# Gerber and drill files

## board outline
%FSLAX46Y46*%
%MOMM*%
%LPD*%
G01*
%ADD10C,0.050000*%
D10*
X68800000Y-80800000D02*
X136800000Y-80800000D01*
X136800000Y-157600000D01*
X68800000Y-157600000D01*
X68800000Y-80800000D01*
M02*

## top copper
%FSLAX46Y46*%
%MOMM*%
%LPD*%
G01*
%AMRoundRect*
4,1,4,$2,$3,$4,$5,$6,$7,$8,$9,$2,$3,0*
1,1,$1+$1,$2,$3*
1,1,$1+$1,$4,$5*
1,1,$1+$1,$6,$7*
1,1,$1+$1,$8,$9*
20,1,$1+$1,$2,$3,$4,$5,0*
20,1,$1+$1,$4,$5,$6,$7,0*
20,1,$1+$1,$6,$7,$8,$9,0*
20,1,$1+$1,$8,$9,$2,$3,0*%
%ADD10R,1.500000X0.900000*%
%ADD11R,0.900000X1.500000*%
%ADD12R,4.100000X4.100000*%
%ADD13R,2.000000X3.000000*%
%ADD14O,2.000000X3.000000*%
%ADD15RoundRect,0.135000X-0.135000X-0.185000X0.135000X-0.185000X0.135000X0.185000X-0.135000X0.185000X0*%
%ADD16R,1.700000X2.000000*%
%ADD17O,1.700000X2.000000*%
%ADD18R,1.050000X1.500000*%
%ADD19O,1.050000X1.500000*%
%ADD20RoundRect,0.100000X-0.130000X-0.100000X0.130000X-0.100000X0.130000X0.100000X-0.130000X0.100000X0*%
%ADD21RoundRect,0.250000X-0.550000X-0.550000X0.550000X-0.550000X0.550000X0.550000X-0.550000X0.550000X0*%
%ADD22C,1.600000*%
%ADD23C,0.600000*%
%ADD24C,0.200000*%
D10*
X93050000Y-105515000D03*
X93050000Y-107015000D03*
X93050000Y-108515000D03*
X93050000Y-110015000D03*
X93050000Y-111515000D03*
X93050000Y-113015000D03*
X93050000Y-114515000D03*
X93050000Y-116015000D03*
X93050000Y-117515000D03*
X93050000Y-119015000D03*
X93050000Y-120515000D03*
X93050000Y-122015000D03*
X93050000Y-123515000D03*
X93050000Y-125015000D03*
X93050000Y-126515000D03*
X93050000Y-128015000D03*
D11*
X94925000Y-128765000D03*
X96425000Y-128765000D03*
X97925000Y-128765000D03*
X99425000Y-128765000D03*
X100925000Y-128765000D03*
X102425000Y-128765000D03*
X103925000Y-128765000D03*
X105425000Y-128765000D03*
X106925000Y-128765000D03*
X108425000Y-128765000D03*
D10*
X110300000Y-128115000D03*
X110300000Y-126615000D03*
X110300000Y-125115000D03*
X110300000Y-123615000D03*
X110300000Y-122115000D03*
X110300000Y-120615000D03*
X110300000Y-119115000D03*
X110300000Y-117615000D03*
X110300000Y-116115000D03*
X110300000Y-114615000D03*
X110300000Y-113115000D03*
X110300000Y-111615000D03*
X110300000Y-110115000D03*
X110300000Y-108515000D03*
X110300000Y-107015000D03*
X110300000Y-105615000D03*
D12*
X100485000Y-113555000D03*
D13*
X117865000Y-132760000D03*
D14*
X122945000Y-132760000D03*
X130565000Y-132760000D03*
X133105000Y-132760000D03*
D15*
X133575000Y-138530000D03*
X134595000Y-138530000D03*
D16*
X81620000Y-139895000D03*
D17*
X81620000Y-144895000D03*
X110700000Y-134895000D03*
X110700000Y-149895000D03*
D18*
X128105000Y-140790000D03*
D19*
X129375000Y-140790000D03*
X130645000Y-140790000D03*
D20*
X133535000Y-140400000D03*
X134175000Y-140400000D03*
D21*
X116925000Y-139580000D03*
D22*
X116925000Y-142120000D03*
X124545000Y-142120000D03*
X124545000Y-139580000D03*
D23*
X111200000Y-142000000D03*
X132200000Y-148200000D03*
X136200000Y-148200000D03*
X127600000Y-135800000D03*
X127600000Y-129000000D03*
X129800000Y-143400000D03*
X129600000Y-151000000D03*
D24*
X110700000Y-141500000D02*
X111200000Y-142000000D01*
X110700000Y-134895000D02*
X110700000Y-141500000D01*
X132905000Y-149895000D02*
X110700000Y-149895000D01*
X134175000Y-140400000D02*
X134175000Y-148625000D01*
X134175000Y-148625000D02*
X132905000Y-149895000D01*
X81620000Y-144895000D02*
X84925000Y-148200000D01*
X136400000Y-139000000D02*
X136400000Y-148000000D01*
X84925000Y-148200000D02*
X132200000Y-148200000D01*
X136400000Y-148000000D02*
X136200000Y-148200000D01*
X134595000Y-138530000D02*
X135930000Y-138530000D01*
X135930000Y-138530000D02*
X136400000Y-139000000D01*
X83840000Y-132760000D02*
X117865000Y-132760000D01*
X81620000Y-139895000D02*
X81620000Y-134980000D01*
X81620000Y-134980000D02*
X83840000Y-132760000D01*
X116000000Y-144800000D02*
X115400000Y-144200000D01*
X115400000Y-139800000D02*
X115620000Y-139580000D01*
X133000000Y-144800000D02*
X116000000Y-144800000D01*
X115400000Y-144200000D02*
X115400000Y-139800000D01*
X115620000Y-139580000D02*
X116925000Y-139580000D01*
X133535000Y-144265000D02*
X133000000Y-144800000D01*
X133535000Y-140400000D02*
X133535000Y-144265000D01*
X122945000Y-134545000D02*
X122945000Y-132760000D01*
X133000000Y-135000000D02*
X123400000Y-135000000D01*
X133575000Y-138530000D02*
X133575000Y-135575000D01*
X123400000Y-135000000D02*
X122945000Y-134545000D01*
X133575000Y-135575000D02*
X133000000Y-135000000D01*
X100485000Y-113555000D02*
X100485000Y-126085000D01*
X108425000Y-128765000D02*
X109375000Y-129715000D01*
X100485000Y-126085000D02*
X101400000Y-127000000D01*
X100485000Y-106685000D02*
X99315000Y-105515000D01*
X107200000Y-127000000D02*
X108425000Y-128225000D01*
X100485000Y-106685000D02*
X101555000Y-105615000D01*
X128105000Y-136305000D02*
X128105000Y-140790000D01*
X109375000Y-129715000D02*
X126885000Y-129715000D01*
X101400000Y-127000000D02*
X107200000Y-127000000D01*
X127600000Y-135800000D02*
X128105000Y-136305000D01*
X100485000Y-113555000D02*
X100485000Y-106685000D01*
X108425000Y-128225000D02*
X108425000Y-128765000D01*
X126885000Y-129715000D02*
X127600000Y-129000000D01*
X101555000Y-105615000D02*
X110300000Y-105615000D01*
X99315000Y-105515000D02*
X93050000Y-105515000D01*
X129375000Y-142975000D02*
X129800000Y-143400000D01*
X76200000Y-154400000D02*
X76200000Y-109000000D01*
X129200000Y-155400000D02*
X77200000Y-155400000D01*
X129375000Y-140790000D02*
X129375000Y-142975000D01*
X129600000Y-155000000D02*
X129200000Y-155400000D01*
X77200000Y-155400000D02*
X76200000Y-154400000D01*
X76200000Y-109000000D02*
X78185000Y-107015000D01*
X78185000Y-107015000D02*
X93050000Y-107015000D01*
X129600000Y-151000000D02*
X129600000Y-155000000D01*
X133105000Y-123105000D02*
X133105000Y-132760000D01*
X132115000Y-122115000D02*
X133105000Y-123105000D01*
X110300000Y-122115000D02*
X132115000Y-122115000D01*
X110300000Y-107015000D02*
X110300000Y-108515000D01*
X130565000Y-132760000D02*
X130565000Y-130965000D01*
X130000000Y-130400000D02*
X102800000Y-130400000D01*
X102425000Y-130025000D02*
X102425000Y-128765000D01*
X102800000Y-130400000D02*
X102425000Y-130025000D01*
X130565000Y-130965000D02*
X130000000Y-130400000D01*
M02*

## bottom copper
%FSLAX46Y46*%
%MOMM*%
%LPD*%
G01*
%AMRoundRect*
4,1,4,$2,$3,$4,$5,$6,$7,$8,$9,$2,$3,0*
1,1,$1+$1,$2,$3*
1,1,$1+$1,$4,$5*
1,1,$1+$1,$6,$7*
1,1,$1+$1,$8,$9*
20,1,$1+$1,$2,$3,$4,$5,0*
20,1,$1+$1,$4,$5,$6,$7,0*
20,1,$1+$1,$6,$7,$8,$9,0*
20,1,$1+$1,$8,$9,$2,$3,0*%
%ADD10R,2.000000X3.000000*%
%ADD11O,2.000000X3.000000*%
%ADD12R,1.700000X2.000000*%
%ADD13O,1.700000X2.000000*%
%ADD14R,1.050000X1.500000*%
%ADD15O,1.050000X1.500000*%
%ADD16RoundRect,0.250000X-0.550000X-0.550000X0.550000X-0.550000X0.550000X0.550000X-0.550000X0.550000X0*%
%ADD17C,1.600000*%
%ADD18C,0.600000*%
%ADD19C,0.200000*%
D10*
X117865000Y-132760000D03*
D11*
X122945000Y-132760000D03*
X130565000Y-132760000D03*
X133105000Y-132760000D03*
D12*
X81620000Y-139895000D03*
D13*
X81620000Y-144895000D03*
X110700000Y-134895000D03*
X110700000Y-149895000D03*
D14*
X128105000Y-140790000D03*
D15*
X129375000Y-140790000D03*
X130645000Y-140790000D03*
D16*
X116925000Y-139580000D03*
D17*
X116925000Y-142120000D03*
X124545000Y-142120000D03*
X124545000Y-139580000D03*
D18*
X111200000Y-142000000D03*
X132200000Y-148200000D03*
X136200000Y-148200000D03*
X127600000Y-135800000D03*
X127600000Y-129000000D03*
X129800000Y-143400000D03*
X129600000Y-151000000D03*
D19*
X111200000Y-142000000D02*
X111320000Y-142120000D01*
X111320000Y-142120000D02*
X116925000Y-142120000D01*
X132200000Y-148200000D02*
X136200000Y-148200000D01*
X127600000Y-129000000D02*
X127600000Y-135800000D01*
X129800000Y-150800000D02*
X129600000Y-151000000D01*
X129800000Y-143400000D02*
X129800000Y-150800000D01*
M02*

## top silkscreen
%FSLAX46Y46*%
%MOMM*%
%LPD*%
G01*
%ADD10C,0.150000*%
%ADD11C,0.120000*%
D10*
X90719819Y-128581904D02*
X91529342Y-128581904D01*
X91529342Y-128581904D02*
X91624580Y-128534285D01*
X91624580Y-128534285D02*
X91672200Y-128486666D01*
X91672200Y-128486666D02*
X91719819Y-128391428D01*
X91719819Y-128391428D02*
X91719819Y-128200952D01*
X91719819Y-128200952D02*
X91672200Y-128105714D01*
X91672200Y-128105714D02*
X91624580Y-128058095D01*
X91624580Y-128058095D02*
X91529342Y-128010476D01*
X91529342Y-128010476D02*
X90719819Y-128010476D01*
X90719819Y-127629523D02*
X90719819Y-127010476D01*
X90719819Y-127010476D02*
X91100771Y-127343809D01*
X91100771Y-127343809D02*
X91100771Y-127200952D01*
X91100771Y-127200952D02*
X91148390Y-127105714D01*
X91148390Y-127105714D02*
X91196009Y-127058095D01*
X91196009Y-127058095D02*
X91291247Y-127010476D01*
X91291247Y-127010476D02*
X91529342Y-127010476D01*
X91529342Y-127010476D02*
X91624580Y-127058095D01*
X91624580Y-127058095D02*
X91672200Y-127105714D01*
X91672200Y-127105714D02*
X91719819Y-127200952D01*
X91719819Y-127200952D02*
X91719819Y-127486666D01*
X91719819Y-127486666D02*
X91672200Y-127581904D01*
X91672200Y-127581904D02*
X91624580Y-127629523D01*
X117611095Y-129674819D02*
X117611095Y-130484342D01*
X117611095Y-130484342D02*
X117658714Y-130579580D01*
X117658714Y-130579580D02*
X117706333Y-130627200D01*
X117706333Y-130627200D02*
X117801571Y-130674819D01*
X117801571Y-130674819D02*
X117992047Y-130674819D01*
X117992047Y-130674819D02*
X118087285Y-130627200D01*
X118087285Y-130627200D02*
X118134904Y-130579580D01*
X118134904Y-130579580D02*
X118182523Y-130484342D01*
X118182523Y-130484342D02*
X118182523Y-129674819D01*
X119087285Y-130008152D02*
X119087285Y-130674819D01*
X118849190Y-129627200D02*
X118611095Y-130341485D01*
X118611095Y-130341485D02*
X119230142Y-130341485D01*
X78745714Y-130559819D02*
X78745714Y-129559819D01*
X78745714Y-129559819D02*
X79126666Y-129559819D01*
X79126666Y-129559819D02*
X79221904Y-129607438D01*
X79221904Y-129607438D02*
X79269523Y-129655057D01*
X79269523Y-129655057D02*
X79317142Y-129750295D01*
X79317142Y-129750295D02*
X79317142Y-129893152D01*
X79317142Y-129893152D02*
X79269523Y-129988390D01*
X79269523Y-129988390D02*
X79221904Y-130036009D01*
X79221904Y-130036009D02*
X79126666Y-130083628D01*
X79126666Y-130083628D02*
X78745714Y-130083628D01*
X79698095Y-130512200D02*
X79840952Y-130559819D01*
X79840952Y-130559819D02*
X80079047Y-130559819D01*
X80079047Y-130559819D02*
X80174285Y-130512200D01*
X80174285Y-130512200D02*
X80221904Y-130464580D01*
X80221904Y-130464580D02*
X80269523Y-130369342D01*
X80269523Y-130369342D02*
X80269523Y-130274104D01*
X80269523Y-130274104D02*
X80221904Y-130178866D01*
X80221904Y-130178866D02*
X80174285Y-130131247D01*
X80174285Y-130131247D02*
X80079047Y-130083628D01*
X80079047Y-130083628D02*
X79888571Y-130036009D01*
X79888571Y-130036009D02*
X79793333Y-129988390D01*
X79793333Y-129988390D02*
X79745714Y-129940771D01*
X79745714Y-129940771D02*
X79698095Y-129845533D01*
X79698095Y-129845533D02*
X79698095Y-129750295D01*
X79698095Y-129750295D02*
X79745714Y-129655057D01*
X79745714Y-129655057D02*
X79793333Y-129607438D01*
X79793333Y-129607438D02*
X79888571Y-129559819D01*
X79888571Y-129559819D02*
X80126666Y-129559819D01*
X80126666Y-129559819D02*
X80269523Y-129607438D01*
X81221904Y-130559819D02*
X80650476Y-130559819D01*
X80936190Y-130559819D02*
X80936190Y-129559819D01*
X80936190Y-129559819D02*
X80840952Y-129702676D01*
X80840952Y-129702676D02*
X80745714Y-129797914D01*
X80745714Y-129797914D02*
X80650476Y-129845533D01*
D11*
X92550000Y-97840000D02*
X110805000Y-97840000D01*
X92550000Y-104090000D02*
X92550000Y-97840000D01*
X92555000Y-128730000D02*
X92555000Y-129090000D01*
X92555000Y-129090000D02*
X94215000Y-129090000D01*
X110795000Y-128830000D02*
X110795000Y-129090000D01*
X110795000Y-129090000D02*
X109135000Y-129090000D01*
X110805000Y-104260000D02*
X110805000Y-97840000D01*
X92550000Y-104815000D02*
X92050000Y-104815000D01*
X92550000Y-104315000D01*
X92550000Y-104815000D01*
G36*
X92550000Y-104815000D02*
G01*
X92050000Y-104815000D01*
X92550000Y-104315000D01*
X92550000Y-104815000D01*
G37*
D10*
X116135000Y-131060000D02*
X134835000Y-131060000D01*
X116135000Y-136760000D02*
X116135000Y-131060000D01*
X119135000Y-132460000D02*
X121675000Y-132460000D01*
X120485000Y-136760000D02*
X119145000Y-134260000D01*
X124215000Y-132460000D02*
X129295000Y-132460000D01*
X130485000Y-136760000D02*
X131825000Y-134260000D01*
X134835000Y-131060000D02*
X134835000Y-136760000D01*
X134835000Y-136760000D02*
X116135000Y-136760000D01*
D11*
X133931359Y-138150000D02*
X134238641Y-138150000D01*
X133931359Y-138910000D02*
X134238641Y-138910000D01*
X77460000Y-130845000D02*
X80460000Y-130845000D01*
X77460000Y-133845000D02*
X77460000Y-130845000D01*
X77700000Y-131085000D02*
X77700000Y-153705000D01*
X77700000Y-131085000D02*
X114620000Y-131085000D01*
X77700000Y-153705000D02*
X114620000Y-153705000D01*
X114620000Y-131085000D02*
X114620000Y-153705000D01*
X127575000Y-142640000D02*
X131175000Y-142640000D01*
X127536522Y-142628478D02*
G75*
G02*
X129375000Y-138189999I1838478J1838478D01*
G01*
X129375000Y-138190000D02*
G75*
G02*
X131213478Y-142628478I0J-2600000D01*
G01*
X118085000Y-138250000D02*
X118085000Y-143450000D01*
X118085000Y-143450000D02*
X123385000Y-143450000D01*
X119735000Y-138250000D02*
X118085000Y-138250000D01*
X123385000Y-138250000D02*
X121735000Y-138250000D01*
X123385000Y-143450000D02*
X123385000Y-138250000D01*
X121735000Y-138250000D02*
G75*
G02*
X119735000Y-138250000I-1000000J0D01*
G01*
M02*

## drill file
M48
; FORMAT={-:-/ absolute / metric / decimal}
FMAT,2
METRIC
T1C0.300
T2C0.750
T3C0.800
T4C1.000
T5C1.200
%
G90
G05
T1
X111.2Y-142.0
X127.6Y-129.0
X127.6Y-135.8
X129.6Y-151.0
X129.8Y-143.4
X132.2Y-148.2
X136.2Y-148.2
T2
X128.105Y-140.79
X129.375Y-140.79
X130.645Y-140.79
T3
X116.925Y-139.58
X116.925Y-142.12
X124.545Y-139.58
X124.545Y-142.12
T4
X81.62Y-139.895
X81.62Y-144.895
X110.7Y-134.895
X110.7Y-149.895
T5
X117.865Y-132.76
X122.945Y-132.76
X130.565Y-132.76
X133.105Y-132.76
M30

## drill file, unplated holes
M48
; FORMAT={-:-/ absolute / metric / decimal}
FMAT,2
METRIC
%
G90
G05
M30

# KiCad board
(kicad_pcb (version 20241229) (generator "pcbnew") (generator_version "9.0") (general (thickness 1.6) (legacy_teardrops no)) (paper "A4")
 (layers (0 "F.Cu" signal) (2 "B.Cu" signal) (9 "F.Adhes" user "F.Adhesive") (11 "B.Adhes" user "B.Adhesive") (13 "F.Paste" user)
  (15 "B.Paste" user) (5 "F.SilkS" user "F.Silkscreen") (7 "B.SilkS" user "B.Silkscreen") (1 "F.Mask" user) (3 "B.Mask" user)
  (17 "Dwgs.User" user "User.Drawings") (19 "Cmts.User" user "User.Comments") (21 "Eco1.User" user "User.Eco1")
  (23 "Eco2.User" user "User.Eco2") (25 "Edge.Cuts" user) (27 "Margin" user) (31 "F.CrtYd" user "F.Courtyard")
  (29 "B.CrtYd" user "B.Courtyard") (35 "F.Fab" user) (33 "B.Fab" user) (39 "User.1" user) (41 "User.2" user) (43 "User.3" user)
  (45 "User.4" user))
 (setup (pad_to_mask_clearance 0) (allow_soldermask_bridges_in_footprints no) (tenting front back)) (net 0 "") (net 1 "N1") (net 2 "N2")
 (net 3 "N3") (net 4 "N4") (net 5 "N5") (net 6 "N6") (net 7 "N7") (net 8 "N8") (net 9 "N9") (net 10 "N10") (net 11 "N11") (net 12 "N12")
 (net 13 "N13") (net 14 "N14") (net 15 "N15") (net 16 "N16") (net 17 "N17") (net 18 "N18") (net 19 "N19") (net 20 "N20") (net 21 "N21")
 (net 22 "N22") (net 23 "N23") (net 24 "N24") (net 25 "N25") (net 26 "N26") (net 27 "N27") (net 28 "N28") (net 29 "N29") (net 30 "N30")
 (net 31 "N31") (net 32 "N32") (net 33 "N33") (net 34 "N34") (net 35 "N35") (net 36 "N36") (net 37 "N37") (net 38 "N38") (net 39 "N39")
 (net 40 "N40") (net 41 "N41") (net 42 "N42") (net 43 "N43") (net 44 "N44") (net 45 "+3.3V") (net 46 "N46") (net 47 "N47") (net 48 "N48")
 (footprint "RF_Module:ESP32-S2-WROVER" (layer "F.Cu") (at 101.675 117.29)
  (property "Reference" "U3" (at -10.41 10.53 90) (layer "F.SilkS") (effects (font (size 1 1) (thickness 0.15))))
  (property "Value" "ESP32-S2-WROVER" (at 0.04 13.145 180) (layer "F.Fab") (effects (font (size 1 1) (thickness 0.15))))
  (fp_line (start -9.125 -19.45) (end 9.13 -19.45) (stroke (width 0.12) (type solid)) (layer "F.SilkS"))
  (fp_line (start -9.125 -13.2) (end -9.125 -19.45) (stroke (width 0.12) (type solid)) (layer "F.SilkS"))
  (fp_line (start -9.12 11.44) (end -9.12 11.8) (stroke (width 0.12) (type solid)) (layer "F.SilkS"))
  (fp_line (start -9.12 11.8) (end -7.46 11.8) (stroke (width 0.12) (type solid)) (layer "F.SilkS"))
  (fp_line (start 9.12 11.54) (end 9.12 11.8) (stroke (width 0.12) (type solid)) (layer "F.SilkS"))
  (fp_line (start 9.12 11.8) (end 7.46 11.8) (stroke (width 0.12) (type solid)) (layer "F.SilkS"))
  (fp_line (start 9.13 -13.03) (end 9.13 -19.45) (stroke (width 0.12) (type solid)) (layer "F.SilkS"))
  (fp_poly
   (pts (xy -9.125 -12.475) (xy -9.625 -12.475) (xy -9.125 -12.975) (xy -9.125 -12.475)) (stroke (width 0.12) (type solid)) (fill yes)
   (layer "F.SilkS"))
  (pad "" smd roundrect (at -2.52 -5.065) (size 1.07 1.07) (layers "F.Paste") (roundrect_rratio 0.233645))
  (pad "" smd roundrect (at -2.52 -3.735) (size 1.07 1.07) (layers "F.Paste") (roundrect_rratio 0.233645))
  (pad "" smd roundrect (at -2.52 -2.405) (size 1.07 1.07) (layers "F.Paste") (roundrect_rratio 0.233645))
  (pad "" smd roundrect (at -1.19 -5.065) (size 1.07 1.07) (layers "F.Paste") (roundrect_rratio 0.233645))
  (pad "" smd roundrect (at -1.19 -3.735) (size 1.07 1.07) (layers "F.Paste") (roundrect_rratio 0.233645))
  (pad "" smd roundrect (at -1.19 -2.405) (size 1.07 1.07) (layers "F.Paste") (roundrect_rratio 0.233645))
  (pad "" smd roundrect (at 0.14 -5.065) (size 1.07 1.07) (layers "F.Paste") (roundrect_rratio 0.233645))
  (pad "" smd roundrect (at 0.14 -3.735) (size 1.07 1.07) (layers "F.Paste") (roundrect_rratio 0.233645))
  (pad "" smd roundrect (at 0.14 -2.405) (size 1.07 1.07) (layers "F.Paste") (roundrect_rratio 0.233645))
  (pad "1" smd rect (at -8.625 -11.775) (size 1.5 0.9) (layers "F.Cu" "F.Mask" "F.Paste") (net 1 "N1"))
  (pad "2" smd rect (at -8.625 -10.275) (size 1.5 0.9) (layers "F.Cu" "F.Mask" "F.Paste") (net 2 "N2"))
  (pad "3" smd rect (at -8.625 -8.775) (size 1.5 0.9) (layers "F.Cu" "F.Mask" "F.Paste") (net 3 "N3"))
  (pad "4" smd rect (at -8.625 -7.275) (size 1.5 0.9) (layers "F.Cu" "F.Mask" "F.Paste") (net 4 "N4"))
  (pad "5" smd rect (at -8.625 -5.775) (size 1.5 0.9) (layers "F.Cu" "F.Mask" "F.Paste") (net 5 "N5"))
  (pad "6" smd rect (at -8.625 -4.275) (size 1.5 0.9) (layers "F.Cu" "F.Mask" "F.Paste") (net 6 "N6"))
  (pad "7" smd rect (at -8.625 -2.775) (size 1.5 0.9) (layers "F.Cu" "F.Mask" "F.Paste") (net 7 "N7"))
  (pad "8" smd rect (at -8.625 -1.275) (size 1.5 0.9) (layers "F.Cu" "F.Mask" "F.Paste") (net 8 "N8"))
  (pad "9" smd rect (at -8.625 0.225) (size 1.5 0.9) (layers "F.Cu" "F.Mask" "F.Paste") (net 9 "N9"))
  (pad "10" smd rect (at -8.625 1.725) (size 1.5 0.9) (layers "F.Cu" "F.Mask" "F.Paste") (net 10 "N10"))
  (pad "11" smd rect (at -8.625 3.225) (size 1.5 0.9) (layers "F.Cu" "F.Mask" "F.Paste") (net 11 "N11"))
  (pad "12" smd rect (at -8.625 4.725) (size 1.5 0.9) (layers "F.Cu" "F.Mask" "F.Paste") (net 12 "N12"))
  (pad "13" smd rect (at -8.625 6.225) (size 1.5 0.9) (layers "F.Cu" "F.Mask" "F.Paste") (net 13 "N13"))
  (pad "14" smd rect (at -8.625 7.725) (size 1.5 0.9) (layers "F.Cu" "F.Mask" "F.Paste") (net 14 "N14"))
  (pad "15" smd rect (at -8.625 9.225 180) (size 1.5 0.9) (layers "F.Cu" "F.Mask" "F.Paste") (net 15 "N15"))
  (pad "16" smd rect (at -8.625 10.725 180) (size 1.5 0.9) (layers "F.Cu" "F.Mask" "F.Paste") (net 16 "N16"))
  (pad "17" smd rect (at -6.75 11.475) (size 0.9 1.5) (layers "F.Cu" "F.Mask" "F.Paste") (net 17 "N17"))
  (pad "18" smd rect (at -5.25 11.475) (size 0.9 1.5) (layers "F.Cu" "F.Mask" "F.Paste") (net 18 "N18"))
  (pad "19" smd rect (at -3.75 11.475) (size 0.9 1.5) (layers "F.Cu" "F.Mask" "F.Paste") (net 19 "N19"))
  (pad "20" smd rect (at -2.25 11.475) (size 0.9 1.5) (layers "F.Cu" "F.Mask" "F.Paste") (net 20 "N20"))
  (pad "21" smd rect (at -0.75 11.475) (size 0.9 1.5) (layers "F.Cu" "F.Mask" "F.Paste") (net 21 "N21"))
  (pad "22" smd rect (at 0.75 11.475) (size 0.9 1.5) (layers "F.Cu" "F.Mask" "F.Paste") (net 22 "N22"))
  (pad "23" smd rect (at 2.25 11.475) (size 0.9 1.5) (layers "F.Cu" "F.Mask" "F.Paste") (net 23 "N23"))
  (pad "24" smd rect (at 3.75 11.475) (size 0.9 1.5) (layers "F.Cu" "F.Mask" "F.Paste") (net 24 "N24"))
  (pad "25" smd rect (at 5.25 11.475) (size 0.9 1.5) (layers "F.Cu" "F.Mask" "F.Paste") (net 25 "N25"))
  (pad "26" smd rect (at 6.75 11.475) (size 0.9 1.5) (layers "F.Cu" "F.Mask" "F.Paste") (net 1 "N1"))
  (pad "27" smd rect (at 8.625 10.825) (size 1.5 0.9) (layers "F.Cu" "F.Mask" "F.Paste") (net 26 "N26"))
  (pad "28" smd rect (at 8.625 9.325) (size 1.5 0.9) (layers "F.Cu" "F.Mask" "F.Paste") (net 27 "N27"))
  (pad "29" smd rect (at 8.625 7.825) (size 1.5 0.9) (layers "F.Cu" "F.Mask" "F.Paste") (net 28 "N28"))
  (pad "30" smd rect (at 8.625 6.325) (size 1.5 0.9) (layers "F.Cu" "F.Mask" "F.Paste") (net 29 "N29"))
  (pad "31" smd rect (at 8.625 4.825) (size 1.5 0.9) (layers "F.Cu" "F.Mask" "F.Paste") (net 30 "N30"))
  (pad "32" smd rect (at 8.625 3.325) (size 1.5 0.9) (layers "F.Cu" "F.Mask" "F.Paste") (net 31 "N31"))
  (pad "33" smd rect (at 8.625 1.825) (size 1.5 0.9) (layers "F.Cu" "F.Mask" "F.Paste") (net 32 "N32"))
  (pad "34" smd rect (at 8.625 0.325) (size 1.5 0.9) (layers "F.Cu" "F.Mask" "F.Paste") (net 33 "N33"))
  (pad "35" smd rect (at 8.625 -1.175) (size 1.5 0.9) (layers "F.Cu" "F.Mask" "F.Paste") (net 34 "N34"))
  (pad "36" smd rect (at 8.625 -2.675) (size 1.5 0.9) (layers "F.Cu" "F.Mask" "F.Paste") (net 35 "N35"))
  (pad "37" smd rect (at 8.625 -4.175) (size 1.5 0.9) (layers "F.Cu" "F.Mask" "F.Paste") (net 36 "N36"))
  (pad "38" smd rect (at 8.625 -5.675) (size 1.5 0.9) (layers "F.Cu" "F.Mask" "F.Paste") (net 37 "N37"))
  (pad "39" smd rect (at 8.625 -7.175) (size 1.5 0.9) (layers "F.Cu" "F.Mask" "F.Paste") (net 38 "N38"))
  (pad "40" smd rect (at 8.625 -8.775) (size 1.5 0.9) (layers "F.Cu" "F.Mask" "F.Paste") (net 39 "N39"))
  (pad "41" smd rect (at 8.625 -10.275) (size 1.5 0.9) (layers "F.Cu" "F.Mask" "F.Paste") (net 39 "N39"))
  (pad "42" smd rect (at 8.625 -11.675) (size 1.5 0.9) (layers "F.Cu" "F.Mask" "F.Paste") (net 1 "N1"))
  (pad "43" smd rect (at -1.19 -3.735) (size 4.1 4.1) (layers "F.Cu" "F.Mask") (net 1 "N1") (zone_connect 2))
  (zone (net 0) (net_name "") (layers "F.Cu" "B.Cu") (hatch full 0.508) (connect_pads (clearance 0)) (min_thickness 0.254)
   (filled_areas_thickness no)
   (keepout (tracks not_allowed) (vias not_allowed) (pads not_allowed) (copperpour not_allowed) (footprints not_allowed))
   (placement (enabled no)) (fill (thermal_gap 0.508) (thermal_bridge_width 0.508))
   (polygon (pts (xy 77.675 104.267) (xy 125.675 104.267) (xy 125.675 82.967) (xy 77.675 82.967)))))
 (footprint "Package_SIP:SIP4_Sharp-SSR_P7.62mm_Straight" (layer "F.Cu") (at 117.865 132.76)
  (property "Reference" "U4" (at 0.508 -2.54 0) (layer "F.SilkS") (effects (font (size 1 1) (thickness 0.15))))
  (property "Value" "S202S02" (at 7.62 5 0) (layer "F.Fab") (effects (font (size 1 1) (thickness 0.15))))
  (fp_line (start -1.73 -1.7) (end 16.97 -1.7) (stroke (width 0.15) (type solid)) (layer "F.SilkS"))
  (fp_line (start -1.73 4) (end -1.73 -1.7) (stroke (width 0.15) (type solid)) (layer "F.SilkS"))
  (fp_line (start 1.27 -0.3) (end 3.81 -0.3) (stroke (width 0.15) (type solid)) (layer "F.SilkS"))
  (fp_line (start 2.62 4) (end 1.28 1.5) (stroke (width 0.15) (type solid)) (layer "F.SilkS"))
  (fp_line (start 6.35 -0.3) (end 11.43 -0.3) (stroke (width 0.15) (type solid)) (layer "F.SilkS"))
  (fp_line (start 12.62 4) (end 13.96 1.5) (stroke (width 0.15) (type solid)) (layer "F.SilkS"))
  (fp_line (start 16.97 -1.7) (end 16.97 4) (stroke (width 0.15) (type solid)) (layer "F.SilkS"))
  (fp_line (start 16.97 4) (end -1.73 4) (stroke (width 0.15) (type solid)) (layer "F.SilkS"))
  (pad "1" thru_hole rect (at 0 0) (size 2 3) (drill 1.2) (layers "*.Cu" "*.Mask") (remove_unused_layers no) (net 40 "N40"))
  (pad "2" thru_hole oval (at 5.08 0) (size 2 3) (drill 1.2) (layers "*.Cu" "*.Mask") (remove_unused_layers no) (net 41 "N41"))
  (pad "3" thru_hole oval (at 12.7 0) (size 2 3) (drill 1.2) (layers "*.Cu" "*.Mask") (remove_unused_layers no) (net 22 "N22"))
  (pad "4" thru_hole oval (at 15.24 0) (size 2 3) (drill 1.2) (layers "*.Cu" "*.Mask") (remove_unused_layers no) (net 30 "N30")))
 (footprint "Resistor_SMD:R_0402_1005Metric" (layer "F.Cu") (at 134.085 138.53)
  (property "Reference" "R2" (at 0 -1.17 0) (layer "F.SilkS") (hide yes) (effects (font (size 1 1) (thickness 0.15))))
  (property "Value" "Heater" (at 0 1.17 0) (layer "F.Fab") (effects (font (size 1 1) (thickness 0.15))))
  (fp_line (start -0.153641 -0.38) (end 0.153641 -0.38) (stroke (width 0.12) (type solid)) (layer "F.SilkS"))
  (fp_line (start -0.153641 0.38) (end 0.153641 0.38) (stroke (width 0.12) (type solid)) (layer "F.SilkS"))
  (pad "1" smd roundrect (at -0.51 0) (size 0.54 0.64) (layers "F.Cu" "F.Mask" "F.Paste") (roundrect_rratio 0.25) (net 41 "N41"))
  (pad "2" smd roundrect (at 0.51 0) (size 0.54 0.64) (layers "F.Cu" "F.Mask" "F.Paste") (roundrect_rratio 0.25) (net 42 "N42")))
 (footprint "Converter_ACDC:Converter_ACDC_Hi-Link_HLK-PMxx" (layer "F.Cu") (at 81.62 139.895)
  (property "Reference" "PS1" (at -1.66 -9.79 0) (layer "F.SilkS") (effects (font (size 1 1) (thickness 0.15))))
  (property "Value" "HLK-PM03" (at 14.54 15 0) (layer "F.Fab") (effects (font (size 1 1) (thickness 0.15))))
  (fp_line (start -4.16 -9.05) (end -1.16 -9.05) (stroke (width 0.12) (type solid)) (layer "F.SilkS"))
  (fp_line (start -4.16 -6.05) (end -4.16 -9.05) (stroke (width 0.12) (type solid)) (layer "F.SilkS"))
  (fp_line (start -3.92 -8.81) (end -3.92 13.81) (stroke (width 0.12) (type solid)) (layer "F.SilkS"))
  (fp_line (start -3.92 -8.81) (end 33 -8.81) (stroke (width 0.12) (type solid)) (layer "F.SilkS"))
  (fp_line (start -3.92 13.81) (end 33 13.81) (stroke (width 0.12) (type solid)) (layer "F.SilkS"))
  (fp_line (start 33 -8.81) (end 33 13.81) (stroke (width 0.12) (type solid)) (layer "F.SilkS"))
  (pad "1" thru_hole rect (at 0 0) (size 1.7 2) (drill 1) (layers "*.Cu" "*.Mask") (remove_unused_layers no) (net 40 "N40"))
  (pad "2" thru_hole oval (at 0 5) (size 1.7 2) (drill 1) (layers "*.Cu" "*.Mask") (remove_unused_layers no) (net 42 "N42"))
  (pad "3" thru_hole oval (at 29.08 -5) (size 1.7 2) (drill 1) (layers "*.Cu" "*.Mask") (remove_unused_layers no) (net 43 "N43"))
  (pad "4" thru_hole oval (at 29.08 10) (size 1.7 2) (drill 1) (layers "*.Cu" "*.Mask") (remove_unused_layers no) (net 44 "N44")))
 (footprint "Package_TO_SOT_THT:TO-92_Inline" (layer "F.Cu") (at 128.105 140.79)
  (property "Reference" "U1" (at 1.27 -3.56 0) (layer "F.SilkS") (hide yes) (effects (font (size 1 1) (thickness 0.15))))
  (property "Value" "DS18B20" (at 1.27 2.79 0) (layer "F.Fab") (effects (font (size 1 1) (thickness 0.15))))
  (fp_line (start -0.53 1.85) (end 3.07 1.85) (stroke (width 0.12) (type solid)) (layer "F.SilkS"))
  (fp_arc (start -0.568478 1.838478) (mid -1.132087 -0.994977) (end 1.27 -2.6) (stroke (width 0.12) (type solid)) (layer "F.SilkS"))
  (fp_arc (start 1.27 -2.6) (mid 3.672087 -0.994977) (end 3.108478 1.838478) (stroke (width 0.12) (type solid)) (layer "F.SilkS"))
  (pad "1" thru_hole rect (at 0 0) (size 1.05 1.5) (drill 0.75) (layers "*.Cu" "*.Mask") (remove_unused_layers no) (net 1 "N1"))
  (pad "2" thru_hole oval (at 1.27 0) (size 1.05 1.5) (drill 0.75) (layers "*.Cu" "*.Mask") (remove_unused_layers no) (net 2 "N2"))
  (pad "3" thru_hole oval (at 2.54 0) (size 1.05 1.5) (drill 0.75) (layers "*.Cu" "*.Mask") (remove_unused_layers no) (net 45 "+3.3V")))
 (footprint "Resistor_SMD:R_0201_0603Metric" (layer "F.Cu") (at 133.855 140.4)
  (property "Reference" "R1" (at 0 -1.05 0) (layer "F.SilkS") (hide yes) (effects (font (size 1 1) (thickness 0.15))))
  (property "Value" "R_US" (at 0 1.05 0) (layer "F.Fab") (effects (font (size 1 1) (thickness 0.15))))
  (pad "" smd roundrect (at -0.345 0) (size 0.318 0.36) (layers "F.Paste") (roundrect_rratio 0.25))
  (pad "" smd roundrect (at 0.345 0) (size 0.318 0.36) (layers "F.Paste") (roundrect_rratio 0.25))
  (pad "1" smd roundrect (at -0.32 0) (size 0.46 0.4) (layers "F.Cu" "F.Mask") (roundrect_rratio 0.25) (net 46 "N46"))
  (pad "2" smd roundrect (at 0.32 0) (size 0.46 0.4) (layers "F.Cu" "F.Mask") (roundrect_rratio 0.25) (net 44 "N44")))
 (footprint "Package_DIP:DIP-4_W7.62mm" (layer "F.Cu") (at 116.925 139.58)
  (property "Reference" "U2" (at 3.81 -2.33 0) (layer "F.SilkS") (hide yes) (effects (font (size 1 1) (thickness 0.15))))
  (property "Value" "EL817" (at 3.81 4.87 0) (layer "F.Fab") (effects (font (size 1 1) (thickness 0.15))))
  (fp_line (start 1.16 -1.33) (end 1.16 3.87) (stroke (width 0.12) (type solid)) (layer "F.SilkS"))
  (fp_line (start 1.16 3.87) (end 6.46 3.87) (stroke (width 0.12) (type solid)) (layer "F.SilkS"))
  (fp_line (start 2.81 -1.33) (end 1.16 -1.33) (stroke (width 0.12) (type solid)) (layer "F.SilkS"))
  (fp_line (start 6.46 -1.33) (end 4.81 -1.33) (stroke (width 0.12) (type solid)) (layer "F.SilkS"))
  (fp_line (start 6.46 3.87) (end 6.46 -1.33) (stroke (width 0.12) (type solid)) (layer "F.SilkS"))
  (fp_arc (start 4.81 -1.33) (mid 3.81 -0.33) (end 2.81 -1.33) (stroke (width 0.12) (type solid)) (layer "F.SilkS"))
  (pad "1" thru_hole roundrect (at 0 0) (size 1.6 1.6) (drill 0.8) (layers "*.Cu" "*.Mask") (remove_unused_layers no)
   (roundrect_rratio 0.15625) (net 46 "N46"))
  (pad "2" thru_hole circle (at 0 2.54) (size 1.6 1.6) (drill 0.8) (layers "*.Cu" "*.Mask") (remove_unused_layers no) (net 43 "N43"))
  (pad "3" thru_hole circle (at 7.62 2.54) (size 1.6 1.6) (drill 0.8) (layers "*.Cu" "*.Mask") (remove_unused_layers no) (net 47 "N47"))
  (pad "4" thru_hole circle (at 7.62 0) (size 1.6 1.6) (drill 0.8) (layers "*.Cu" "*.Mask") (remove_unused_layers no) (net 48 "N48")))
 (gr_rect (start 68.8 80.8) (end 136.8 157.6) (stroke (width 0.05) (type default)) (fill no) (layer "Edge.Cuts"))
 (segment (start 110.7 141.5) (end 111.2 142) (width 0.2) (layer "F.Cu") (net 43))
 (segment (start 110.7 134.895) (end 110.7 141.5) (width 0.2) (layer "F.Cu") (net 43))
 (via (at 111.2 142) (size 0.6) (drill 0.3) (layers "F.Cu" "B.Cu") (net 43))
 (segment (start 111.2 142) (end 111.32 142.12) (width 0.2) (layer "B.Cu") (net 43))
 (segment (start 111.32 142.12) (end 116.925 142.12) (width 0.2) (layer "B.Cu") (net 43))
 (segment (start 132.905 149.895) (end 110.7 149.895) (width 0.2) (layer "F.Cu") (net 44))
 (segment (start 134.175 140.4) (end 134.175 148.625) (width 0.2) (layer "F.Cu") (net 44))
 (segment (start 134.175 148.625) (end 132.905 149.895) (width 0.2) (layer "F.Cu") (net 44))
 (segment (start 81.62 144.895) (end 84.925 148.2) (width 0.2) (layer "F.Cu") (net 42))
 (segment (start 136.4 139) (end 136.4 148) (width 0.2) (layer "F.Cu") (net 42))
 (segment (start 84.925 148.2) (end 132.2 148.2) (width 0.2) (layer "F.Cu") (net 42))
 (segment (start 136.4 148) (end 136.2 148.2) (width 0.2) (layer "F.Cu") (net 42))
 (segment (start 134.595 138.53) (end 135.93 138.53) (width 0.2) (layer "F.Cu") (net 42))
 (segment (start 135.93 138.53) (end 136.4 139) (width 0.2) (layer "F.Cu") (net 42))
 (via (at 132.2 148.2) (size 0.6) (drill 0.3) (layers "F.Cu" "B.Cu") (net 42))
 (via (at 136.2 148.2) (size 0.6) (drill 0.3) (layers "F.Cu" "B.Cu") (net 42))
 (segment (start 132.2 148.2) (end 136.2 148.2) (width 0.2) (layer "B.Cu") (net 42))
 (segment (start 83.84 132.76) (end 117.865 132.76) (width 0.2) (layer "F.Cu") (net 40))
 (segment (start 81.62 139.895) (end 81.62 134.98) (width 0.2) (layer "F.Cu") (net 40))
 (segment (start 81.62 134.98) (end 83.84 132.76) (width 0.2) (layer "F.Cu") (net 40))
 (segment (start 116 144.8) (end 115.4 144.2) (width 0.2) (layer "F.Cu") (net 46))
 (segment (start 115.4 139.8) (end 115.62 139.58) (width 0.2) (layer "F.Cu") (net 46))
 (segment (start 133 144.8) (end 116 144.8) (width 0.2) (layer "F.Cu") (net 46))
 (segment (start 115.4 144.2) (end 115.4 139.8) (width 0.2) (layer "F.Cu") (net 46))
 (segment (start 115.62 139.58) (end 116.925 139.58) (width 0.2) (layer "F.Cu") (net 46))
 (segment (start 133.535 144.265) (end 133 144.8) (width 0.2) (layer "F.Cu") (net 46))
 (segment (start 133.535 140.4) (end 133.535 144.265) (width 0.2) (layer "F.Cu") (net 46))
 (segment (start 122.945 134.545) (end 122.945 132.76) (width 0.2) (layer "F.Cu") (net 41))
 (segment (start 133 135) (end 123.4 135) (width 0.2) (layer "F.Cu") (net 41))
 (segment (start 133.575 138.53) (end 133.575 135.575) (width 0.2) (layer "F.Cu") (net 41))
 (segment (start 123.4 135) (end 122.945 134.545) (width 0.2) (layer "F.Cu") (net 41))
 (segment (start 133.575 135.575) (end 133 135) (width 0.2) (layer "F.Cu") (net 41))
 (segment (start 100.485 113.555) (end 100.485 126.085) (width 0.2) (layer "F.Cu") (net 1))
 (segment (start 108.425 128.765) (end 109.375 129.715) (width 0.2) (layer "F.Cu") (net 1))
 (segment (start 100.485 126.085) (end 101.4 127) (width 0.2) (layer "F.Cu") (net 1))
 (segment (start 100.485 106.685) (end 99.315 105.515) (width 0.2) (layer "F.Cu") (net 1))
 (segment (start 107.2 127) (end 108.425 128.225) (width 0.2) (layer "F.Cu") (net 1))
 (segment (start 100.485 106.685) (end 101.555 105.615) (width 0.2) (layer "F.Cu") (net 1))
 (segment (start 128.105 136.305) (end 128.105 140.79) (width 0.2) (layer "F.Cu") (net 1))
 (segment (start 109.375 129.715) (end 126.885 129.715) (width 0.2) (layer "F.Cu") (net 1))
 (segment (start 101.4 127) (end 107.2 127) (width 0.2) (layer "F.Cu") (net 1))
 (segment (start 127.6 135.8) (end 128.105 136.305) (width 0.2) (layer "F.Cu") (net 1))
 (segment (start 100.485 113.555) (end 100.485 106.685) (width 0.2) (layer "F.Cu") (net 1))
 (segment (start 108.425 128.225) (end 108.425 128.765) (width 0.2) (layer "F.Cu") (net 1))
 (segment (start 126.885 129.715) (end 127.6 129) (width 0.2) (layer "F.Cu") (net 1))
 (segment (start 101.555 105.615) (end 110.3 105.615) (width 0.2) (layer "F.Cu") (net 1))
 (segment (start 99.315 105.515) (end 93.05 105.515) (width 0.2) (layer "F.Cu") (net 1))
 (via (at 127.6 135.8) (size 0.6) (drill 0.3) (layers "F.Cu" "B.Cu") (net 1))
 (via (at 127.6 129) (size 0.6) (drill 0.3) (layers "F.Cu" "B.Cu") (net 1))
 (segment (start 127.6 129) (end 127.6 135.8) (width 0.2) (layer "B.Cu") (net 1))
 (segment (start 129.375 142.975) (end 129.8 143.4) (width 0.2) (layer "F.Cu") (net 2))
 (segment (start 76.2 154.4) (end 76.2 109) (width 0.2) (layer "F.Cu") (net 2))
 (segment (start 129.2 155.4) (end 77.2 155.4) (width 0.2) (layer "F.Cu") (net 2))
 (segment (start 129.375 140.79) (end 129.375 142.975) (width 0.2) (layer "F.Cu") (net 2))
 (segment (start 129.6 155) (end 129.2 155.4) (width 0.2) (layer "F.Cu") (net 2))
 (segment (start 77.2 155.4) (end 76.2 154.4) (width 0.2) (layer "F.Cu") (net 2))
 (segment (start 76.2 109) (end 78.185 107.015) (width 0.2) (layer "F.Cu") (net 2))
 (segment (start 78.185 107.015) (end 93.05 107.015) (width 0.2) (layer "F.Cu") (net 2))
 (segment (start 129.6 151) (end 129.6 155) (width 0.2) (layer "F.Cu") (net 2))
 (via (at 129.8 143.4) (size 0.6) (drill 0.3) (layers "F.Cu" "B.Cu") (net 2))
 (via (at 129.6 151) (size 0.6) (drill 0.3) (layers "F.Cu" "B.Cu") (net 2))
 (segment (start 129.8 150.8) (end 129.6 151) (width 0.2) (layer "B.Cu") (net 2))
 (segment (start 129.8 143.4) (end 129.8 150.8) (width 0.2) (layer "B.Cu") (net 2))
 (segment (start 133.105 123.105) (end 133.105 132.76) (width 0.2) (layer "F.Cu") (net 30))
 (segment (start 132.115 122.115) (end 133.105 123.105) (width 0.2) (layer "F.Cu") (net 30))
 (segment (start 110.3 122.115) (end 132.115 122.115) (width 0.2) (layer "F.Cu") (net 30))
 (segment (start 110.3 107.015) (end 110.3 108.515) (width 0.2) (layer "F.Cu") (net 39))
 (segment (start 130.565 132.76) (end 130.565 130.965) (width 0.2) (layer "F.Cu") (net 22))
 (segment (start 130 130.4) (end 102.8 130.4) (width 0.2) (layer "F.Cu") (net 22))
 (segment (start 102.425 130.025) (end 102.425 128.765) (width 0.2) (layer "F.Cu") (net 22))
 (segment (start 102.8 130.4) (end 102.425 130.025) (width 0.2) (layer "F.Cu") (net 22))
 (segment (start 130.565 130.965) (end 130 130.4) (width 0.2) (layer "F.Cu") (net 22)))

